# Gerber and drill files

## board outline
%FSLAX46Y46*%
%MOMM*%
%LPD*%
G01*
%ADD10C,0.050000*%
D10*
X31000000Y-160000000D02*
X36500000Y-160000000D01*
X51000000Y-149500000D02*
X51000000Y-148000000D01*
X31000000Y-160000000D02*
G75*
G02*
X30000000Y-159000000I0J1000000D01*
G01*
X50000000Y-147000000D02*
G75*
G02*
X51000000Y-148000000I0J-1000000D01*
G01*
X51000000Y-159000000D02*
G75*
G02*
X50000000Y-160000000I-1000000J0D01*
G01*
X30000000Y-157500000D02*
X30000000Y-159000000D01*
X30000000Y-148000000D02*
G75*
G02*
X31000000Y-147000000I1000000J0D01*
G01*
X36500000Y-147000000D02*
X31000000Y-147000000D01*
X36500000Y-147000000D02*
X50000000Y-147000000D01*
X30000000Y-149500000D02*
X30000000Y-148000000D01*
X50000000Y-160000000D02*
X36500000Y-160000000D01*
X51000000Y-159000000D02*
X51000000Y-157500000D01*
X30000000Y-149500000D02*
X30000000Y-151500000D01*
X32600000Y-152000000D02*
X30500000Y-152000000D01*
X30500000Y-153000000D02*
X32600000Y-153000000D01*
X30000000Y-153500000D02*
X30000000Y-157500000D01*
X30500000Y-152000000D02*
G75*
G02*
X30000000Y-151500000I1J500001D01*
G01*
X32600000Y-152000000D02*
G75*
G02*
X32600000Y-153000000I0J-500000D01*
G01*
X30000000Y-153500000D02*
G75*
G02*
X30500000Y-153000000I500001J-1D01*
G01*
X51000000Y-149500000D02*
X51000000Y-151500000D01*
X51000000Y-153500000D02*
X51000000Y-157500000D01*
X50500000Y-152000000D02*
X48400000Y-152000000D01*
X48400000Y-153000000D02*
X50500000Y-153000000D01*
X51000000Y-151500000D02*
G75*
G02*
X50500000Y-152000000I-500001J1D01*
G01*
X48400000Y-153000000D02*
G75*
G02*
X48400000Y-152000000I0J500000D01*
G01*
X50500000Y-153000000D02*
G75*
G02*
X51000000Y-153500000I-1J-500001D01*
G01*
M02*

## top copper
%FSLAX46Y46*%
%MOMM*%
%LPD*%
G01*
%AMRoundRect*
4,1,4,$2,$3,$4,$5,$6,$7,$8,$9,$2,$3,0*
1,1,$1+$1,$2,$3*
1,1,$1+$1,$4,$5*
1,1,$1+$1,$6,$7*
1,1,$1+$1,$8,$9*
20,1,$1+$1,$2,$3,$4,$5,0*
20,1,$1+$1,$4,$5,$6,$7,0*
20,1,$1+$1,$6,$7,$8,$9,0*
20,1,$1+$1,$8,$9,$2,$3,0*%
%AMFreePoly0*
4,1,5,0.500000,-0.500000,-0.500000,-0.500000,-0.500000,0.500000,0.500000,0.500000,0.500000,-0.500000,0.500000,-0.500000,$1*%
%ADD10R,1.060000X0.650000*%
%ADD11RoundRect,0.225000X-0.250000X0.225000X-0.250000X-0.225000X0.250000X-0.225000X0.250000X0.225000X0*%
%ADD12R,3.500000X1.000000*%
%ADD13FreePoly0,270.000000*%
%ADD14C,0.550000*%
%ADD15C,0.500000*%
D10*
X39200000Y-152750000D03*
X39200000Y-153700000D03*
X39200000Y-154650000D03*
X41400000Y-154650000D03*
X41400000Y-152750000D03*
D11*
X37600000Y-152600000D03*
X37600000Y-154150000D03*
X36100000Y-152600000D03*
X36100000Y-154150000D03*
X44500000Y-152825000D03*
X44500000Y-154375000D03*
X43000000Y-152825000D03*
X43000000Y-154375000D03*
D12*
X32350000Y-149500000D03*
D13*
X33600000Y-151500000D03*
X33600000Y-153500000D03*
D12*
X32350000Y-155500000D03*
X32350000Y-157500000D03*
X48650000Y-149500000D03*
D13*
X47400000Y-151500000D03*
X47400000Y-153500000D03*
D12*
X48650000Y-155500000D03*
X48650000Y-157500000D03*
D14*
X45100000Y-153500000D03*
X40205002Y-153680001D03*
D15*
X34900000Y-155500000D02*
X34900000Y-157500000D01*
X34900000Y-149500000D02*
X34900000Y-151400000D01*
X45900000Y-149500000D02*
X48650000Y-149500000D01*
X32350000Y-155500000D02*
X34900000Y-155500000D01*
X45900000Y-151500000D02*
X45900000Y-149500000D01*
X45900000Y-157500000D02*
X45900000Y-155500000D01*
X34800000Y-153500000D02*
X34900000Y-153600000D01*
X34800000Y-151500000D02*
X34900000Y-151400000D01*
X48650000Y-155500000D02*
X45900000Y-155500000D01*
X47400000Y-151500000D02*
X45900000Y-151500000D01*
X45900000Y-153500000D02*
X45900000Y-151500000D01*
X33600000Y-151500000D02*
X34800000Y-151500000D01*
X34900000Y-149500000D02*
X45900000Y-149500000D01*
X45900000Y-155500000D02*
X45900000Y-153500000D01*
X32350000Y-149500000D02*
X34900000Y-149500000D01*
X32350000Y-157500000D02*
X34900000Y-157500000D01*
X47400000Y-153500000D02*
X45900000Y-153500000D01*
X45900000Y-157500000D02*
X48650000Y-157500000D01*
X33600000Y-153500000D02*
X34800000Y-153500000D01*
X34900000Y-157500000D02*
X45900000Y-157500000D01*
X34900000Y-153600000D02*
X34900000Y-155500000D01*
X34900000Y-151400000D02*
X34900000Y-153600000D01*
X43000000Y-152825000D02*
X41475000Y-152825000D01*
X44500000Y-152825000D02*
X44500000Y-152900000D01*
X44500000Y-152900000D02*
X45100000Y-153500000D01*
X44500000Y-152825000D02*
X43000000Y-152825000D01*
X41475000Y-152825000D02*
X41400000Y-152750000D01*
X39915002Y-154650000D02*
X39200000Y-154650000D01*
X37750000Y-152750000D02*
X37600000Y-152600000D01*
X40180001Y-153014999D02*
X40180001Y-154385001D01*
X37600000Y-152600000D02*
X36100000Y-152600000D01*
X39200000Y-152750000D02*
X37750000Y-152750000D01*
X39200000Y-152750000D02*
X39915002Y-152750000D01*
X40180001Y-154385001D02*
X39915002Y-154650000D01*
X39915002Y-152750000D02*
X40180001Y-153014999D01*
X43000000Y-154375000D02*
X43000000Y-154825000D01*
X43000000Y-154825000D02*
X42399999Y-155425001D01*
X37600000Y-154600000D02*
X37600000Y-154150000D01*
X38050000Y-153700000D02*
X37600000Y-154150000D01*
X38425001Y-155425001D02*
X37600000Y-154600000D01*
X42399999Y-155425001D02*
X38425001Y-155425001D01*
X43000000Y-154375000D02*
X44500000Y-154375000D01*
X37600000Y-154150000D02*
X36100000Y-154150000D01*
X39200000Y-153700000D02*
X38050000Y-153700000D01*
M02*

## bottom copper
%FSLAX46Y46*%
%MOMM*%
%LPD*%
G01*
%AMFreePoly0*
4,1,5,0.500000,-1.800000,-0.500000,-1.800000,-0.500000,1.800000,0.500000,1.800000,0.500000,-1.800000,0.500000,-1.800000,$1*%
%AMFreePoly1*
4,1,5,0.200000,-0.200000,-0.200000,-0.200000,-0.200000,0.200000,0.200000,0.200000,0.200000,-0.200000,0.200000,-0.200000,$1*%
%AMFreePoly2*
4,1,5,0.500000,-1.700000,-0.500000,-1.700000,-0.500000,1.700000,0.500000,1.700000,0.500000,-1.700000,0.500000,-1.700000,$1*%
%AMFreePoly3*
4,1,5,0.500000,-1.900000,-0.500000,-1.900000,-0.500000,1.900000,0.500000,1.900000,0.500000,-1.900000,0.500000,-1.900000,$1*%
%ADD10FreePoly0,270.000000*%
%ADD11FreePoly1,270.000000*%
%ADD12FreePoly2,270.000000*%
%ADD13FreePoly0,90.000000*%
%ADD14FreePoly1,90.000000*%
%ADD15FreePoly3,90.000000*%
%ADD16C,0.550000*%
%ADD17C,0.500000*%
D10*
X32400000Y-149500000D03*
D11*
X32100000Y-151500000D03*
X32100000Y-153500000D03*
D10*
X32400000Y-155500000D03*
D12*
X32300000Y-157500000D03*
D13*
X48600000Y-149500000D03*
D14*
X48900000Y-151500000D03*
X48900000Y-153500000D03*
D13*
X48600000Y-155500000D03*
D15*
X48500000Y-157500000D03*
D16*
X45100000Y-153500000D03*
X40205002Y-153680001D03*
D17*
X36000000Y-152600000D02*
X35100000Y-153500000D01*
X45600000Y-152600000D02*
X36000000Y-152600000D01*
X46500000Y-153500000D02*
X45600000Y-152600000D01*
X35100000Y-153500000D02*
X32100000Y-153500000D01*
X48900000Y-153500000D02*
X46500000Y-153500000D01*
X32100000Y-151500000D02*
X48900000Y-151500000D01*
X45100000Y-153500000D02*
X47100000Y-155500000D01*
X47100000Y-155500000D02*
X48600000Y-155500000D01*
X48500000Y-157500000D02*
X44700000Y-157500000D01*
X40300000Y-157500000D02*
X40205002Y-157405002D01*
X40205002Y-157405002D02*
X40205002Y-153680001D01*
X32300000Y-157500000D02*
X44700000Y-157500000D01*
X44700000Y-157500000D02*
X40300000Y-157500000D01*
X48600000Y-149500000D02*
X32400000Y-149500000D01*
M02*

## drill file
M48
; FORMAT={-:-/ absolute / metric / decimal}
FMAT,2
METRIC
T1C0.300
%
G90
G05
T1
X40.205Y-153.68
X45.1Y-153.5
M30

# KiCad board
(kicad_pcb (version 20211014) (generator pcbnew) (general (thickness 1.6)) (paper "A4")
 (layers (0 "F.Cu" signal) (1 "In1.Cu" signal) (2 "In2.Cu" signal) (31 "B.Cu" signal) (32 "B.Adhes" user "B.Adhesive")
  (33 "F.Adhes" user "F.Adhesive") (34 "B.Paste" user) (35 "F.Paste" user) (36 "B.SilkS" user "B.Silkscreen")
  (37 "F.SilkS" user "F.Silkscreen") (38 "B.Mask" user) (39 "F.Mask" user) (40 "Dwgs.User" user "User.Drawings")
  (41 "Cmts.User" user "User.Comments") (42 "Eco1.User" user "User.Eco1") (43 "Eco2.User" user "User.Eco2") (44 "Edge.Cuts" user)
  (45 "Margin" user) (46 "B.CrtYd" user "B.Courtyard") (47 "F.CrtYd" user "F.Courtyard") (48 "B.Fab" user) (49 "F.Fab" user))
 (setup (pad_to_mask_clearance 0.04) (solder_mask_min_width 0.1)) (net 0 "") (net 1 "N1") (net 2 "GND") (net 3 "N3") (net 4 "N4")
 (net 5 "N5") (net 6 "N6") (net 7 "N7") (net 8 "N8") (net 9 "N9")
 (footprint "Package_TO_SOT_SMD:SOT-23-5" (layer "F.Cu") (at 40.3 153.7)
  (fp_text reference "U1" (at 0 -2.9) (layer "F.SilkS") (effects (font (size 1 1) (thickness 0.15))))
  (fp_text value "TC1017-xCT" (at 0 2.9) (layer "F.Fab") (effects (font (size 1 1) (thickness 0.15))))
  (pad "1" smd rect locked (at -1.1 -0.95) (size 1.06 0.65) (layers "F.Cu" "F.Paste" "F.Mask") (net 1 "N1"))
  (pad "2" smd rect locked (at -1.1 0) (size 1.06 0.65) (layers "F.Cu" "F.Paste" "F.Mask") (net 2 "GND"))
  (pad "3" smd rect locked (at -1.1 0.95) (size 1.06 0.65) (layers "F.Cu" "F.Paste" "F.Mask") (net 1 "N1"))
  (pad "4" smd rect locked (at 1.1 0.95) (size 1.06 0.65) (layers "F.Cu" "F.Paste" "F.Mask") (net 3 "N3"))
  (pad "5" smd rect locked (at 1.1 -0.95) (size 1.06 0.65) (layers "F.Cu" "F.Paste" "F.Mask") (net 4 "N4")))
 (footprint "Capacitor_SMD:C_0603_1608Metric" (layer "F.Cu") (at 37.6 153.375 -90)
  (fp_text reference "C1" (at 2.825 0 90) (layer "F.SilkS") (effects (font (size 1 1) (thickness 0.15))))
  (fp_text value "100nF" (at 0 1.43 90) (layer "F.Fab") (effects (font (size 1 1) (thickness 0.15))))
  (pad "1" smd roundrect locked (at -0.775 0 270) (size 0.9 0.95) (layers "F.Cu" "F.Paste" "F.Mask") (roundrect_rratio 0.25) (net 1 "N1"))
  (pad "2" smd roundrect locked (at 0.775 0 270) (size 0.9 0.95) (layers "F.Cu" "F.Paste" "F.Mask") (roundrect_rratio 0.25) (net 2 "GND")))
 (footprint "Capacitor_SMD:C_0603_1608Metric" (layer "F.Cu") (at 36.1 153.375 -90)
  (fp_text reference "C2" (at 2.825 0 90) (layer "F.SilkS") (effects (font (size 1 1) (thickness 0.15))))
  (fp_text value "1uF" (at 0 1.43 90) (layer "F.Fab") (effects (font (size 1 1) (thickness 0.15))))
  (pad "1" smd roundrect locked (at -0.775 0 270) (size 0.9 0.95) (layers "F.Cu" "F.Paste" "F.Mask") (roundrect_rratio 0.25) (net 1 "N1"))
  (pad "2" smd roundrect locked (at 0.775 0 270) (size 0.9 0.95) (layers "F.Cu" "F.Paste" "F.Mask") (roundrect_rratio 0.25) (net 2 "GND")))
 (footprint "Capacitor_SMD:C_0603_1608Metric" (layer "F.Cu") (at 44.5 153.6 -90)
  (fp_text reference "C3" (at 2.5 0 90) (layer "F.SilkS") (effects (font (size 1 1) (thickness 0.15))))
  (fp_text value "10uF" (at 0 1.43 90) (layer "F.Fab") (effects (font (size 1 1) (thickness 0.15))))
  (pad "1" smd roundrect locked (at -0.775 0 270) (size 0.9 0.95) (layers "F.Cu" "F.Paste" "F.Mask") (roundrect_rratio 0.25) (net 4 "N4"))
  (pad "2" smd roundrect locked (at 0.775 0 270) (size 0.9 0.95) (layers "F.Cu" "F.Paste" "F.Mask") (roundrect_rratio 0.25) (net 2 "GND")))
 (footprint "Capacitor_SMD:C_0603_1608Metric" (layer "F.Cu") (at 43 153.6 -90)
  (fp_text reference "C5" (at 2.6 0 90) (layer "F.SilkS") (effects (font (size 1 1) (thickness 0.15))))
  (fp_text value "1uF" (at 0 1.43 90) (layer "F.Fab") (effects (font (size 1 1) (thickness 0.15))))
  (pad "1" smd roundrect locked (at -0.775 0 270) (size 0.9 0.95) (layers "F.Cu" "F.Paste" "F.Mask") (roundrect_rratio 0.25) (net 4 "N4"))
  (pad "2" smd roundrect locked (at 0.775 0 270) (size 0.9 0.95) (layers "F.Cu" "F.Paste" "F.Mask") (roundrect_rratio 0.25) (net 2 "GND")))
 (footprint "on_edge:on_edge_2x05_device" (layer "F.Cu") (at 30 153.5 -90)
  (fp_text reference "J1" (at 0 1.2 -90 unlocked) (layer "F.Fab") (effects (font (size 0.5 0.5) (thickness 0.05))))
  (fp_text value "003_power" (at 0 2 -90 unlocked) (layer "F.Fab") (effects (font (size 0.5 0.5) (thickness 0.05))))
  (fp_line (start -4 0) (end -2 0) (layer "Edge.Cuts") (width 0.05))
  (fp_line (start -1.5 -2.6) (end -1.5 -0.5) (layer "Edge.Cuts") (width 0.05))
  (fp_line (start -0.5 -0.5) (end -0.5 -2.6) (layer "Edge.Cuts") (width 0.05))
  (fp_line (start 0 0) (end 4 0) (layer "Edge.Cuts") (width 0.05))
  (fp_arc (start -1.5 -0.5) (mid -1.646447 -0.146447) (end -2 0) (layer "Edge.Cuts") (width 0.05))
  (fp_arc (start -1.5 -2.6) (mid -1 -3.1) (end -0.5 -2.6) (layer "Edge.Cuts") (width 0.05))
  (fp_arc (start 0 0) (mid -0.353553 -0.146447) (end -0.5 -0.5) (layer "Edge.Cuts") (width 0.05))
  (pad "1" smd rect locked (at -4 -2.35 90) (size 1 3.5) (layers "F.Cu" "F.Mask") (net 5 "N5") (zone_connect 0))
  (pad "2" smd custom locked (at -2 -3.6 270) (size 1 1) (layers "F.Cu" "F.Mask") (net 5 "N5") (zone_connect 0)
   (options (clearance outline) (anchor rect)) (primitives))
  (pad "3" smd custom locked (at 0 -3.6 270) (size 1 1) (layers "F.Cu" "F.Mask") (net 5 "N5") (zone_connect 0)
   (options (clearance outline) (anchor rect)) (primitives))
  (pad "4" smd rect locked (at 2 -2.35 90) (size 1 3.5) (layers "F.Cu" "F.Mask") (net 5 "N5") (zone_connect 0))
  (pad "5" smd rect locked (at 4 -2.35 90) (size 1 3.5) (layers "F.Cu" "F.Mask") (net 5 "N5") (zone_connect 0))
  (pad "6" smd custom locked (at -4 -2.4 270) (size 1 3.6) (layers "B.Cu" "B.Mask") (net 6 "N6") (zone_connect 0)
   (options (clearance outline) (anchor rect)) (primitives))
  (pad "7" smd custom locked (at -2 -2.1 270) (size 0.4 0.4) (layers "B.Cu" "B.Mask") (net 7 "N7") (zone_connect 0)
   (options (clearance outline) (anchor rect)) (primitives))
  (pad "8" smd custom locked (at 0 -2.1 270) (size 0.4 0.4) (layers "B.Cu" "B.Mask") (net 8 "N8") (zone_connect 0)
   (options (clearance outline) (anchor rect)) (primitives))
  (pad "9" smd custom locked (at 2 -2.4 270) (size 1 3.6) (layers "B.Cu" "B.Mask") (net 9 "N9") (zone_connect 0)
   (options (clearance outline) (anchor rect)) (primitives))
  (pad "10" smd custom locked (at 4 -2.3 270) (size 1 3.4) (layers "B.Cu" "B.Mask") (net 1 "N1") (zone_connect 0)
   (options (clearance outline) (anchor rect)) (primitives)))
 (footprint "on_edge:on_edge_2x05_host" (layer "F.Cu") (at 51 153.5 -90)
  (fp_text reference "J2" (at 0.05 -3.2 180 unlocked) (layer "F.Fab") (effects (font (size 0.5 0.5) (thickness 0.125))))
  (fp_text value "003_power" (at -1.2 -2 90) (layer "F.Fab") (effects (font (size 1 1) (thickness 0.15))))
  (fp_line (start -4 0) (end -2 0) (layer "Edge.Cuts") (width 0.05))
  (fp_line (start 0 0) (end 4 0) (layer "Edge.Cuts") (width 0.05))
  (fp_line (start -1.5 0.5) (end -1.5 2.6) (layer "Edge.Cuts") (width 0.05))
  (fp_line (start -0.5 2.6) (end -0.5 0.5) (layer "Edge.Cuts") (width 0.05))
  (fp_arc (start -2 0) (mid -1.646447 0.146447) (end -1.5 0.5) (layer "Edge.Cuts") (width 0.05))
  (fp_arc (start -0.5 2.6) (mid -1 3.1) (end -1.5 2.6) (layer "Edge.Cuts") (width 0.05))
  (fp_arc (start -0.5 0.5) (mid -0.353553 0.146447) (end 0 0) (layer "Edge.Cuts") (width 0.05))
  (pad "1" smd rect locked (at -4 2.35 270) (size 1 3.5) (layers "F.Cu" "F.Mask") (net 5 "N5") (zone_connect 0))
  (pad "2" smd custom locked (at -2 3.6 270) (size 1 1) (layers "F.Cu" "F.Mask") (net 5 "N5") (zone_connect 0)
   (options (clearance outline) (anchor rect)) (primitives))
  (pad "3" smd custom locked (at 0 3.6 270) (size 1 1) (layers "F.Cu" "F.Mask") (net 5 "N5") (zone_connect 0)
   (options (clearance outline) (anchor rect)) (primitives))
  (pad "4" smd rect locked (at 2 2.35 270) (size 1 3.5) (layers "F.Cu" "F.Mask") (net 5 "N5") (zone_connect 0))
  (pad "5" smd rect locked (at 4 2.35 270) (size 1 3.5) (layers "F.Cu" "F.Mask") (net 5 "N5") (zone_connect 0))
  (pad "6" smd custom locked (at -4 2.4 90) (size 1 3.6) (layers "B.Cu" "B.Mask") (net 6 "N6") (zone_connect 0)
   (options (clearance outline) (anchor rect)) (primitives))
  (pad "7" smd custom locked (at -2 2.1 90) (size 0.4 0.4) (layers "B.Cu" "B.Mask") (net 7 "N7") (zone_connect 0)
   (options (clearance outline) (anchor rect)) (primitives))
  (pad "8" smd custom locked (at 0 2.1 90) (size 0.4 0.4) (layers "B.Cu" "B.Mask") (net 8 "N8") (zone_connect 0)
   (options (clearance outline) (anchor rect)) (primitives))
  (pad "9" smd custom locked (at 2 2.4 90) (size 1 3.6) (layers "B.Cu" "B.Mask") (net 4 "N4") (zone_connect 0)
   (options (clearance outline) (anchor rect)) (primitives))
  (pad "10" smd custom locked (at 4 2.5 90) (size 1 3.8) (layers "B.Cu" "B.Mask") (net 1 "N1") (zone_connect 0)
   (options (clearance outline) (anchor rect)) (primitives)))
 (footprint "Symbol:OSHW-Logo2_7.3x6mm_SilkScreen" (layer "B.Cu") (at 40.4 157.1 180)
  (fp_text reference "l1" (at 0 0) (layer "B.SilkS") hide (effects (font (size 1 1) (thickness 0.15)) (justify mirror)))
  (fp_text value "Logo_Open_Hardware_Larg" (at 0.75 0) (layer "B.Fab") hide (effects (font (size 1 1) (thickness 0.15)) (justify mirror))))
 (gr_line (start 31 160) (end 36.5 160) (layer "Edge.Cuts") (width 0.05))
 (gr_line (start 51 149.5) (end 51 148) (layer "Edge.Cuts") (width 0.05))
 (gr_arc (start 31 160) (mid 30.292893 159.707107) (end 30 159) (layer "Edge.Cuts") (width 0.05))
 (gr_arc (start 50 147) (mid 50.707107 147.292893) (end 51 148) (layer "Edge.Cuts") (width 0.05))
 (gr_arc (start 51 159) (mid 50.707107 159.707107) (end 50 160) (layer "Edge.Cuts") (width 0.05))
 (gr_line (start 30 157.5) (end 30 159) (layer "Edge.Cuts") (width 0.05))
 (gr_arc (start 30 148) (mid 30.292893 147.292893) (end 31 147) (layer "Edge.Cuts") (width 0.05))
 (gr_line (start 36.5 147) (end 31 147) (layer "Edge.Cuts") (width 0.05))
 (gr_line (start 36.5 147) (end 50 147) (layer "Edge.Cuts") (width 0.05))
 (gr_line (start 30 149.5) (end 30 148) (layer "Edge.Cuts") (width 0.05))
 (gr_line (start 50 160) (end 36.5 160) (layer "Edge.Cuts") (width 0.05))
 (gr_line (start 51 159) (end 51 157.5) (layer "Edge.Cuts") (width 0.05))
 (segment (start 34.9 155.5) (end 34.9 157.5) (width 0.5) (layer "F.Cu") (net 5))
 (segment (start 34.9 149.5) (end 34.9 151.4) (width 0.5) (layer "F.Cu") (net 5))
 (segment (start 45.9 149.5) (end 48.65 149.5) (width 0.5) (layer "F.Cu") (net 5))
 (segment (start 32.35 155.5) (end 34.9 155.5) (width 0.5) (layer "F.Cu") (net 5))
 (segment (start 45.9 151.5) (end 45.9 149.5) (width 0.5) (layer "F.Cu") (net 5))
 (segment (start 45.9 157.5) (end 45.9 155.5) (width 0.5) (layer "F.Cu") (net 5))
 (segment (start 34.8 153.5) (end 34.9 153.6) (width 0.5) (layer "F.Cu") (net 5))
 (segment (start 34.8 151.5) (end 34.9 151.4) (width 0.5) (layer "F.Cu") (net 5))
 (segment (start 48.65 155.5) (end 45.9 155.5) (width 0.5) (layer "F.Cu") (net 5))
 (segment (start 47.4 151.5) (end 45.9 151.5) (width 0.5) (layer "F.Cu") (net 5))
 (segment (start 45.9 153.5) (end 45.9 151.5) (width 0.5) (layer "F.Cu") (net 5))
 (segment (start 33.6 151.5) (end 34.8 151.5) (width 0.5) (layer "F.Cu") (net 5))
 (segment (start 34.9 149.5) (end 45.9 149.5) (width 0.5) (layer "F.Cu") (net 5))
 (segment (start 45.9 155.5) (end 45.9 153.5) (width 0.5) (layer "F.Cu") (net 5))
 (segment (start 32.35 149.5) (end 34.9 149.5) (width 0.5) (layer "F.Cu") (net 5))
 (segment (start 32.35 157.5) (end 34.9 157.5) (width 0.5) (layer "F.Cu") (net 5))
 (segment (start 47.4 153.5) (end 45.9 153.5) (width 0.5) (layer "F.Cu") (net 5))
 (segment (start 45.9 157.5) (end 48.65 157.5) (width 0.5) (layer "F.Cu") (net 5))
 (segment (start 33.6 153.5) (end 34.8 153.5) (width 0.5) (layer "F.Cu") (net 5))
 (segment (start 34.9 157.5) (end 45.9 157.5) (width 0.5) (layer "F.Cu") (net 5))
 (segment (start 34.9 153.6) (end 34.9 155.5) (width 0.5) (layer "F.Cu") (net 5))
 (segment (start 34.9 151.4) (end 34.9 153.6) (width 0.5) (layer "F.Cu") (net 5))
 (segment (start 36 152.6) (end 35.1 153.5) (width 0.5) (layer "B.Cu") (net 8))
 (segment (start 45.6 152.6) (end 36 152.6) (width 0.5) (layer "B.Cu") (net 8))
 (segment (start 46.5 153.5) (end 45.6 152.6) (width 0.5) (layer "B.Cu") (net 8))
 (segment (start 35.1 153.5) (end 32.1 153.5) (width 0.5) (layer "B.Cu") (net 8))
 (segment (start 48.9 153.5) (end 46.5 153.5) (width 0.5) (layer "B.Cu") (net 8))
 (segment (start 32.1 151.5) (end 48.9 151.5) (width 0.5) (layer "B.Cu") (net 7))
 (segment (start 43 152.825) (end 41.475 152.825) (width 0.5) (layer "F.Cu") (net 4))
 (segment (start 44.5 152.825) (end 44.5 152.9) (width 0.5) (layer "F.Cu") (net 4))
 (segment (start 44.5 152.9) (end 45.1 153.5) (width 0.5) (layer "F.Cu") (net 4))
 (segment (start 44.5 152.825) (end 43 152.825) (width 0.5) (layer "F.Cu") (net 4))
 (segment (start 41.475 152.825) (end 41.4 152.75) (width 0.5) (layer "F.Cu") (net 4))
 (via (at 45.1 153.5) (size 0.55) (drill 0.3) (layers "F.Cu" "B.Cu") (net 4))
 (segment (start 45.1 153.5) (end 47.1 155.5) (width 0.5) (layer "B.Cu") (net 4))
 (segment (start 47.1 155.5) (end 48.6 155.5) (width 0.5) (layer "B.Cu") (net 4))
 (segment (start 39.915002 154.65) (end 39.2 154.65) (width 0.5) (layer "F.Cu") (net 1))
 (segment (start 37.75 152.75) (end 37.6 152.6) (width 0.5) (layer "F.Cu") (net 1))
 (segment (start 40.180001 153.014999) (end 40.180001 154.385001) (width 0.5) (layer "F.Cu") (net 1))
 (segment (start 37.6 152.6) (end 36.1 152.6) (width 0.5) (layer "F.Cu") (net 1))
 (segment (start 39.2 152.75) (end 37.75 152.75) (width 0.5) (layer "F.Cu") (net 1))
 (segment (start 39.2 152.75) (end 39.915002 152.75) (width 0.5) (layer "F.Cu") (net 1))
 (segment (start 40.180001 154.385001) (end 39.915002 154.65) (width 0.5) (layer "F.Cu") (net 1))
 (segment (start 39.915002 152.75) (end 40.180001 153.014999) (width 0.5) (layer "F.Cu") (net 1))
 (via (at 40.205002 153.680001) (size 0.55) (drill 0.3) (layers "F.Cu" "B.Cu") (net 1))
 (segment (start 48.5 157.5) (end 44.7 157.5) (width 0.5) (layer "B.Cu") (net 1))
 (segment (start 40.3 157.5) (end 40.205002 157.405002) (width 0.5) (layer "B.Cu") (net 1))
 (segment (start 40.205002 157.405002) (end 40.205002 153.680001) (width 0.5) (layer "B.Cu") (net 1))
 (segment (start 32.3 157.5) (end 44.7 157.5) (width 0.5) (layer "B.Cu") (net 1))
 (segment (start 44.7 157.5) (end 40.3 157.5) (width 0.5) (layer "B.Cu") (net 1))
 (segment (start 43 154.375) (end 43 154.825) (width 0.5) (layer "F.Cu") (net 2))
 (segment (start 43 154.825) (end 42.399999 155.425001) (width 0.5) (layer "F.Cu") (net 2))
 (segment (start 37.6 154.6) (end 37.6 154.15) (width 0.5) (layer "F.Cu") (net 2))
 (segment (start 38.05 153.7) (end 37.6 154.15) (width 0.5) (layer "F.Cu") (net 2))
 (segment (start 38.425001 155.425001) (end 37.6 154.6) (width 0.5) (layer "F.Cu") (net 2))
 (segment (start 42.399999 155.425001) (end 38.425001 155.425001) (width 0.5) (layer "F.Cu") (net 2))
 (segment (start 43 154.375) (end 44.5 154.375) (width 0.5) (layer "F.Cu") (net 2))
 (segment (start 37.6 154.15) (end 36.1 154.15) (width 0.5) (layer "F.Cu") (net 2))
 (segment (start 39.2 153.7) (end 38.05 153.7) (width 0.5) (layer "F.Cu") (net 2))
 (segment (start 48.6 149.5) (end 32.4 149.5) (width 0.5) (layer "B.Cu") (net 6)))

